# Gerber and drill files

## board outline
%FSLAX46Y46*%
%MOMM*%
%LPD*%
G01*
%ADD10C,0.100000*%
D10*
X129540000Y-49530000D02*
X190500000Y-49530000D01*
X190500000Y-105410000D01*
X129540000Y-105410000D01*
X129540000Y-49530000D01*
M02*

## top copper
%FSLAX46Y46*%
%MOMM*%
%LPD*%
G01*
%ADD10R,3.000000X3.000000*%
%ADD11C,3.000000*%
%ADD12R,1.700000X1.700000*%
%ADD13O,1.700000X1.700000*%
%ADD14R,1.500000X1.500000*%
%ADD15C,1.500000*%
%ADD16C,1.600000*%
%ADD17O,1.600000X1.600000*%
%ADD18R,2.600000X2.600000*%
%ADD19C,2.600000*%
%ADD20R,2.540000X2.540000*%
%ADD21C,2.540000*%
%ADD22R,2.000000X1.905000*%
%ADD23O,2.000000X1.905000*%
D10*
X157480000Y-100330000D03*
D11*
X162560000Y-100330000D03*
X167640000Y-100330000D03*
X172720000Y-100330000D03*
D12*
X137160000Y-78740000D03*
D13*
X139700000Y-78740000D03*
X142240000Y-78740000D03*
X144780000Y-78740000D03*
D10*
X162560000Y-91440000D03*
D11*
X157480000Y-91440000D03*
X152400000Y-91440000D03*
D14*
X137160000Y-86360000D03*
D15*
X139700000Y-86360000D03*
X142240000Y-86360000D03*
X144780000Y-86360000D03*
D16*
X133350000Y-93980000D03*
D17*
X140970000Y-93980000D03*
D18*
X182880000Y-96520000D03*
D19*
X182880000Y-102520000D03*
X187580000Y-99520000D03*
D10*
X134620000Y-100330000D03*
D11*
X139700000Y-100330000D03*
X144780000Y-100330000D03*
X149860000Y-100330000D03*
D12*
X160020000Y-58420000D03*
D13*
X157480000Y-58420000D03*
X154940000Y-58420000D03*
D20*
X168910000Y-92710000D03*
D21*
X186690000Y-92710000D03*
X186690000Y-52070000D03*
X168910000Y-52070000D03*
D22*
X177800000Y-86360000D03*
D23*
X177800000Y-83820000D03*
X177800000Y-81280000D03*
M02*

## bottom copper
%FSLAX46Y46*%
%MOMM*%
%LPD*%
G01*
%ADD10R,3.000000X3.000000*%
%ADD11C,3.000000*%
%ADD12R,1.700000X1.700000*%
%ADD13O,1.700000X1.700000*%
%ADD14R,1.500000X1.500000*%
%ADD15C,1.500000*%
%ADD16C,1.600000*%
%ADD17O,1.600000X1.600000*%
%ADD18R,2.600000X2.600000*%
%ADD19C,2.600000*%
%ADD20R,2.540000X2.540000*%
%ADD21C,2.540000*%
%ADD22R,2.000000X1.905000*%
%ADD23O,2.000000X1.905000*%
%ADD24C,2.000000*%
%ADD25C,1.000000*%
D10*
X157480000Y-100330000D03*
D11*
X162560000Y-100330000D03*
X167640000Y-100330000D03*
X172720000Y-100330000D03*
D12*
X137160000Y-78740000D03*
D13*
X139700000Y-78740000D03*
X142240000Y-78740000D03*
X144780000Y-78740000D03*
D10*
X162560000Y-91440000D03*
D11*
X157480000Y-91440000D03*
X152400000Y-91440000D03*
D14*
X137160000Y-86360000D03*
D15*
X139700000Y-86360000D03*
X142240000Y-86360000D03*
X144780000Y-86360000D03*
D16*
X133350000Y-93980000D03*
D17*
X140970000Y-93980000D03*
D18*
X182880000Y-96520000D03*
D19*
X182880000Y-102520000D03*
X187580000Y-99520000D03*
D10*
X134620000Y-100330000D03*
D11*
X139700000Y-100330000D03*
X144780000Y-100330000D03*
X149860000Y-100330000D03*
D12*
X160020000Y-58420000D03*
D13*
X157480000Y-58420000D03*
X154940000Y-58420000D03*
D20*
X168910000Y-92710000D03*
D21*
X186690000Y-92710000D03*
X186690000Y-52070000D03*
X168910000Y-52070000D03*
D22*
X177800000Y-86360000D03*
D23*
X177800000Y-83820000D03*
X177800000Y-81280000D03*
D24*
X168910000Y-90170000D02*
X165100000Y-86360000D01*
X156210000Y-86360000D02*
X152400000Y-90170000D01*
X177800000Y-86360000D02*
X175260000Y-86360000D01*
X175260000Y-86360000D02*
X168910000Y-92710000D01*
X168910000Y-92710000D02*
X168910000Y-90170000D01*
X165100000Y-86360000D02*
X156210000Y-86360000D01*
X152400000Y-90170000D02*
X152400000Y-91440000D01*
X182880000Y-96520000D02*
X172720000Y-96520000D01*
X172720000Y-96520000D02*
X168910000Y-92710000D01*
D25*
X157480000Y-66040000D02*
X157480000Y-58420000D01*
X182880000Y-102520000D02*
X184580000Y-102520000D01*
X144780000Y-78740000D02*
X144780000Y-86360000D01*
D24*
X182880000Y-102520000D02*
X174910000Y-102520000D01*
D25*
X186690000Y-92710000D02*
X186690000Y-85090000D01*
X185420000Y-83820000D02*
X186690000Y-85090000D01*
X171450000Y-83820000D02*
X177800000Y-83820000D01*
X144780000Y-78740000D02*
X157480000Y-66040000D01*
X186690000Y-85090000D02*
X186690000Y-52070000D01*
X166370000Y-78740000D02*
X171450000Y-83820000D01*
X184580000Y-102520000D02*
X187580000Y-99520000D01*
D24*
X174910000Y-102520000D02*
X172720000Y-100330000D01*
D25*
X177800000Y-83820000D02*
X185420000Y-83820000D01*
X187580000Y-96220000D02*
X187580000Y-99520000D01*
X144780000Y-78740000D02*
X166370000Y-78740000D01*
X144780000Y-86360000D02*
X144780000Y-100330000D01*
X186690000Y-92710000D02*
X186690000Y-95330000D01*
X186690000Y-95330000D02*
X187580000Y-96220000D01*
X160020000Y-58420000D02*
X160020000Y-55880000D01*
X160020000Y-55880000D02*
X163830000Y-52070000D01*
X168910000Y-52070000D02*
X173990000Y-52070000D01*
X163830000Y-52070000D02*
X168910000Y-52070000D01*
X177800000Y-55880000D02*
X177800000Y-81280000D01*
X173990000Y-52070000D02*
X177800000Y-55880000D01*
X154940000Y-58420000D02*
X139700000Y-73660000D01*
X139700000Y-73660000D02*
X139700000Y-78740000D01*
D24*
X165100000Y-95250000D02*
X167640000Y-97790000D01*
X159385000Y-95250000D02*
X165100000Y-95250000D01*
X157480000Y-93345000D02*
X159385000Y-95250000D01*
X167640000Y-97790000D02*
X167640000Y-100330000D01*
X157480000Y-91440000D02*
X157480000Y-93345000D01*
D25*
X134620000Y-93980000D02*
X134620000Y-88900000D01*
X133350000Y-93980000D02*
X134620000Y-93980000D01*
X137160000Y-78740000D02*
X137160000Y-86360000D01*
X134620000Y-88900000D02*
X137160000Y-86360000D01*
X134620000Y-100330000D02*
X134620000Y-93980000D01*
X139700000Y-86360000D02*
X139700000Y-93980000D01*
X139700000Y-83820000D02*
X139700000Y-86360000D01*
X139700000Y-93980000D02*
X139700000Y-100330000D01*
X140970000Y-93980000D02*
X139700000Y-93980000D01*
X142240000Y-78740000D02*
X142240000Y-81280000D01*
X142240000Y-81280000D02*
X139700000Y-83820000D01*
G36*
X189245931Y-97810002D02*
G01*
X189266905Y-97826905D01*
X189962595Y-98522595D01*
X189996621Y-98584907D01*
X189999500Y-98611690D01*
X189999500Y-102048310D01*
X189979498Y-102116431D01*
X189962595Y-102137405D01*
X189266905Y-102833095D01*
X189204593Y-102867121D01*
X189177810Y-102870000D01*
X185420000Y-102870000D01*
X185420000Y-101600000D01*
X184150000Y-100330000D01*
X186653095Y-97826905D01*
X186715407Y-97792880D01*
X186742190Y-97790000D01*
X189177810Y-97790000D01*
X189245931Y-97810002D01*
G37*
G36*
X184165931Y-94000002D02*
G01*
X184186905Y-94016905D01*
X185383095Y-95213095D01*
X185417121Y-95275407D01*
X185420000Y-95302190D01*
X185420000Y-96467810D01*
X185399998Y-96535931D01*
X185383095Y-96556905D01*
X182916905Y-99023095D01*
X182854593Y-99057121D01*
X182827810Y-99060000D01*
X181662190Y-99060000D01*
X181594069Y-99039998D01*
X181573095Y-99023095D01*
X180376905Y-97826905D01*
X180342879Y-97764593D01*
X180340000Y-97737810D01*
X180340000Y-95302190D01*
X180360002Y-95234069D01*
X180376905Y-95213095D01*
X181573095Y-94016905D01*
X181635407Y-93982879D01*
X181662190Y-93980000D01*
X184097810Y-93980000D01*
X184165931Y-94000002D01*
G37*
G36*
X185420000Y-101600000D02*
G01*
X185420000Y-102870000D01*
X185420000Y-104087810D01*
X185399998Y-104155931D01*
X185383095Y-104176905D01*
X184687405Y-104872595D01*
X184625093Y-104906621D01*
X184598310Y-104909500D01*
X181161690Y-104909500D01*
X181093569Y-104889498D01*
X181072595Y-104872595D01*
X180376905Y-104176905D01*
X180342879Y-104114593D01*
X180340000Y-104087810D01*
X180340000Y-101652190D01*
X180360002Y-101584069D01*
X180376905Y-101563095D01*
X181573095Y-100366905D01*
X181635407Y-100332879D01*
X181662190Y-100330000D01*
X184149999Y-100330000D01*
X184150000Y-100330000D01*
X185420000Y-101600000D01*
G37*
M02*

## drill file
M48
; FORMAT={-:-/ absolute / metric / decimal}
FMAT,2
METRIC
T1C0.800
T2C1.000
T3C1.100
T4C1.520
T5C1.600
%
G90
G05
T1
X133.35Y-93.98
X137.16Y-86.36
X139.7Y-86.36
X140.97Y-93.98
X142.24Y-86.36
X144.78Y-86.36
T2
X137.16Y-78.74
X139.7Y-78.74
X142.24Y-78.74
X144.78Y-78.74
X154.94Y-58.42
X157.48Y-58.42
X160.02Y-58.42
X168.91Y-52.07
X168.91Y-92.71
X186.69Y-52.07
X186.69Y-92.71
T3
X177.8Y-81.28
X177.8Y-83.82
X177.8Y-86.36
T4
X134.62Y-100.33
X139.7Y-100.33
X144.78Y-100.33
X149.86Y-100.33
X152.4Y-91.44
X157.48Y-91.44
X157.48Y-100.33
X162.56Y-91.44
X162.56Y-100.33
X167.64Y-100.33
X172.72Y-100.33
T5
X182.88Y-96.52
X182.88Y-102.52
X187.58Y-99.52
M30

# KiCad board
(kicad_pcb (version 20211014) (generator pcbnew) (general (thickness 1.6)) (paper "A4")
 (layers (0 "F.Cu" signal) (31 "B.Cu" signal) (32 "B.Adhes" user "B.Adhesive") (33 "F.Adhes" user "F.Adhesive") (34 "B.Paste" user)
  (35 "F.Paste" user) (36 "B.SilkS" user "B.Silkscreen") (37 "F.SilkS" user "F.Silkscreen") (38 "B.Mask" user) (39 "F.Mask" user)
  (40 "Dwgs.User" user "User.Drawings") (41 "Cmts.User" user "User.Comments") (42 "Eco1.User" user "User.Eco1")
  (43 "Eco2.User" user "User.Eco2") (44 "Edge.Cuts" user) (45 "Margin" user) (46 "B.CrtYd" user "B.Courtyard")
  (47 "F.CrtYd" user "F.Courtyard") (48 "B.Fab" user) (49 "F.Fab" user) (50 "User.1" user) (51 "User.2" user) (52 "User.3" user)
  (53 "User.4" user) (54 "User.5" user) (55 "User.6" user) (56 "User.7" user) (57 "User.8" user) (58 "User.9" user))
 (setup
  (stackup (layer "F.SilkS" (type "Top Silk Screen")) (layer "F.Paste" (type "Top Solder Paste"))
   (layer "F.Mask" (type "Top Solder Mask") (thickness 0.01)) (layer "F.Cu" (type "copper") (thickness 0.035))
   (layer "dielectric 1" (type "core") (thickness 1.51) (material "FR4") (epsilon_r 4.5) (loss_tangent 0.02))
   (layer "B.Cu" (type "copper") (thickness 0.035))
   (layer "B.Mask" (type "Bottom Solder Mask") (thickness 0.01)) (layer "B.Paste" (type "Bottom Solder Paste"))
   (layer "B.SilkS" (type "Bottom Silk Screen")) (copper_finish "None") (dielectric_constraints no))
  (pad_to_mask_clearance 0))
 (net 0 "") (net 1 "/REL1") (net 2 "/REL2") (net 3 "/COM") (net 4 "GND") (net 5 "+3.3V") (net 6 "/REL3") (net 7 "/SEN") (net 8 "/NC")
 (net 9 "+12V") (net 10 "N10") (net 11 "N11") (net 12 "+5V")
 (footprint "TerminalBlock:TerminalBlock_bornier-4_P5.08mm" (layer "F.Cu") (at 157.48 100.33)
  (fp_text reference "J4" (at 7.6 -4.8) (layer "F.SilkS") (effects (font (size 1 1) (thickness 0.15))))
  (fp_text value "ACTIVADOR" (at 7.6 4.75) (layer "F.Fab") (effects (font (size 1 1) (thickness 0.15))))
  (pad "1" thru_hole rect (at 0 0) (size 3 3) (drill 1.52) (layers *.Cu *.Mask) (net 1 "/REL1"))
  (pad "2" thru_hole circle (at 5.08 0) (size 3 3) (drill 1.52) (layers *.Cu *.Mask) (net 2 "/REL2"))
  (pad "3" thru_hole circle (at 10.16 0) (size 3 3) (drill 1.52) (layers *.Cu *.Mask) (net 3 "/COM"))
  (pad "4" thru_hole circle (at 15.24 0) (size 3 3) (drill 1.52) (layers *.Cu *.Mask) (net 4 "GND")))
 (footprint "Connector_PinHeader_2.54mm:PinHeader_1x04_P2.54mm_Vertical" (layer "F.Cu") (at 137.16 78.74 90)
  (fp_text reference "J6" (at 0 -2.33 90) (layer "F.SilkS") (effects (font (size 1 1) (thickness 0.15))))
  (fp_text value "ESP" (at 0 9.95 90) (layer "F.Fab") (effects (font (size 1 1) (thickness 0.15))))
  (pad "1" thru_hole rect (at 0 0 90) (size 1.7 1.7) (drill 1) (layers *.Cu *.Mask) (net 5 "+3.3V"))
  (pad "2" thru_hole oval (at 0 2.54 90) (size 1.7 1.7) (drill 1) (layers *.Cu *.Mask) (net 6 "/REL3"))
  (pad "3" thru_hole oval (at 0 5.08 90) (size 1.7 1.7) (drill 1) (layers *.Cu *.Mask) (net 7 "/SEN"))
  (pad "4" thru_hole oval (at 0 7.62 90) (size 1.7 1.7) (drill 1) (layers *.Cu *.Mask) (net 4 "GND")))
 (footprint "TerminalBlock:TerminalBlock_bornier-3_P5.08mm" (layer "F.Cu") (at 162.56 91.44 180)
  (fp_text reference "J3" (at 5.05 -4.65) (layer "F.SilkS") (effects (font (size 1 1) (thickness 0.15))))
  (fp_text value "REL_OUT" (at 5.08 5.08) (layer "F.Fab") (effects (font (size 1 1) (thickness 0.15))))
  (pad "1" thru_hole rect (at 0 0 180) (size 3 3) (drill 1.52) (layers *.Cu *.Mask) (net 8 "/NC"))
  (pad "2" thru_hole circle (at 5.08 0 180) (size 3 3) (drill 1.52) (layers *.Cu *.Mask) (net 3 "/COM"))
  (pad "3" thru_hole circle (at 10.16 0 180) (size 3 3) (drill 1.52) (layers *.Cu *.Mask) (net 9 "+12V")))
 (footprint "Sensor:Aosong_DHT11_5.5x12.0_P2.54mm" (layer "F.Cu") (at 137.16 86.36 90)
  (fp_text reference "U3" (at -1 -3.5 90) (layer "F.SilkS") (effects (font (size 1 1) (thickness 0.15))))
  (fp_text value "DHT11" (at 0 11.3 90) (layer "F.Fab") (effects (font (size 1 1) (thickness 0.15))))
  (pad "1" thru_hole rect (at 0 0 90) (size 1.5 1.5) (drill 0.8) (layers *.Cu *.Mask) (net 5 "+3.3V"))
  (pad "2" thru_hole circle (at 0 2.54 90) (size 1.5 1.5) (drill 0.8) (layers *.Cu *.Mask) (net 7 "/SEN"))
  (pad "3" thru_hole circle (at 0 5.08 90) (size 1.5 1.5) (drill 0.8) (layers *.Cu *.Mask) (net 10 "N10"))
  (pad "4" thru_hole circle (at 0 7.62 90) (size 1.5 1.5) (drill 0.8) (layers *.Cu *.Mask) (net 4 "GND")))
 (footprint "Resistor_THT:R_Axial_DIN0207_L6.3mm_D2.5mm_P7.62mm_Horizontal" (layer "F.Cu") (at 133.35 93.98)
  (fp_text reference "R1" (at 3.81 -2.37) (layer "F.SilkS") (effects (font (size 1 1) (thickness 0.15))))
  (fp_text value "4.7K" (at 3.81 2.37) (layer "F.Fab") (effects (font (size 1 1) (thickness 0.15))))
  (pad "1" thru_hole circle (at 0 0) (size 1.6 1.6) (drill 0.8) (layers *.Cu *.Mask) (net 5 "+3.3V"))
  (pad "2" thru_hole oval (at 7.62 0) (size 1.6 1.6) (drill 0.8) (layers *.Cu *.Mask) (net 7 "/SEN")))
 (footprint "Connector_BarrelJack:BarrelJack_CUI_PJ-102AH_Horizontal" (layer "F.Cu") (at 182.88 96.52)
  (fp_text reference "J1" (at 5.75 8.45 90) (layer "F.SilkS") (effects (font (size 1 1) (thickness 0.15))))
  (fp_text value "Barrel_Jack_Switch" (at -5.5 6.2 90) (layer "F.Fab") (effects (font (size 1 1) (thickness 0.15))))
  (pad "1" thru_hole rect (at 0 0) (size 2.6 2.6) (drill 1.6) (layers *.Cu *.Mask) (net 9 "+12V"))
  (pad "2" thru_hole circle (at 0 6) (size 2.6 2.6) (drill 1.6) (layers *.Cu *.Mask) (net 4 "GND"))
  (pad "3" thru_hole circle (at 4.7 3) (size 2.6 2.6) (drill 1.6) (layers *.Cu *.Mask) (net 4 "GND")))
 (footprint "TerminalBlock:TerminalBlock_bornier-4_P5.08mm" (layer "F.Cu") (at 134.62 100.33)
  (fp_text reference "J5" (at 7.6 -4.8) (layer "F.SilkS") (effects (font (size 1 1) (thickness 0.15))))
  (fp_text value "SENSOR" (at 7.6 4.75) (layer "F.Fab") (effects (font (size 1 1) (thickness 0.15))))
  (pad "1" thru_hole rect (at 0 0) (size 3 3) (drill 1.52) (layers *.Cu *.Mask) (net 5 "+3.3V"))
  (pad "2" thru_hole circle (at 5.08 0) (size 3 3) (drill 1.52) (layers *.Cu *.Mask) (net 7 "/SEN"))
  (pad "3" thru_hole circle (at 10.16 0) (size 3 3) (drill 1.52) (layers *.Cu *.Mask) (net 4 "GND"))
  (pad "4" thru_hole circle (at 15.24 0) (size 3 3) (drill 1.52) (layers *.Cu *.Mask) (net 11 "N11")))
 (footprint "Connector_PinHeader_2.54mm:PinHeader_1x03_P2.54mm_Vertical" (layer "F.Cu") (at 160.02 58.42 -90)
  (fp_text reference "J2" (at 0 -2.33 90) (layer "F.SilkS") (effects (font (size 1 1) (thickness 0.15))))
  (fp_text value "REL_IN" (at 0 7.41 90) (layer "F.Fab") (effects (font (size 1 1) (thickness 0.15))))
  (pad "1" thru_hole rect (at 0 0 270) (size 1.7 1.7) (drill 1) (layers *.Cu *.Mask) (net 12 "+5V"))
  (pad "2" thru_hole oval (at 0 2.54 270) (size 1.7 1.7) (drill 1) (layers *.Cu *.Mask) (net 4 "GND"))
  (pad "3" thru_hole oval (at 0 5.08 270) (size 1.7 1.7) (drill 1) (layers *.Cu *.Mask) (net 6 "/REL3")))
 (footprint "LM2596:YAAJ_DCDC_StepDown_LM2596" (layer "F.Cu") (at 168.91 92.71 90)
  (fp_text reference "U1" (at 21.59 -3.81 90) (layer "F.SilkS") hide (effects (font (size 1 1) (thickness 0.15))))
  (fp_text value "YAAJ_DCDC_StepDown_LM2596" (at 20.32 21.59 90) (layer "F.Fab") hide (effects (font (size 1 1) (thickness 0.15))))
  (pad "1" thru_hole rect locked (at 0 0 90) (size 2.54 2.54) (drill 1) (layers *.Cu *.Mask) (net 9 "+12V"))
  (pad "2" thru_hole circle locked (at 0 17.78 90) (size 2.54 2.54) (drill 1) (layers *.Cu *.Mask) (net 4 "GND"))
  (pad "3" thru_hole circle locked (at 40.64 17.78 90) (size 2.54 2.54) (drill 1) (layers *.Cu *.Mask) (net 4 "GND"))
  (pad "4" thru_hole circle locked (at 40.64 0 90) (size 2.54 2.54) (drill 1) (layers *.Cu *.Mask) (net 12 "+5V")))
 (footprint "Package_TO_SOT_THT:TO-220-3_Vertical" (layer "F.Cu") (at 177.8 86.36 90)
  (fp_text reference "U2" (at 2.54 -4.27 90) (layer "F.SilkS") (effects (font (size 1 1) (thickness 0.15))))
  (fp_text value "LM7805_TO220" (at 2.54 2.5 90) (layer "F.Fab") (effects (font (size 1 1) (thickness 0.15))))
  (pad "1" thru_hole rect (at 0 0 90) (size 1.905 2) (drill 1.1) (layers *.Cu *.Mask) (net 9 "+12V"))
  (pad "2" thru_hole oval (at 2.54 0 90) (size 1.905 2) (drill 1.1) (layers *.Cu *.Mask) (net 4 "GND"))
  (pad "3" thru_hole oval (at 5.08 0 90) (size 1.905 2) (drill 1.1) (layers *.Cu *.Mask) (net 12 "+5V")))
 (gr_rect (start 190.5 105.41) (end 129.54 49.53) (layer "Edge.Cuts") (width 0.1) (fill none))
 (segment (start 168.91 90.17) (end 165.1 86.36) (width 2) (layer "B.Cu") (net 9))
 (segment (start 156.21 86.36) (end 152.4 90.17) (width 2) (layer "B.Cu") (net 9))
 (segment (start 177.8 86.36) (end 175.26 86.36) (width 2) (layer "B.Cu") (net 9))
 (segment (start 175.26 86.36) (end 168.91 92.71) (width 2) (layer "B.Cu") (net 9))
 (segment (start 168.91 92.71) (end 168.91 90.17) (width 2) (layer "B.Cu") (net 9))
 (segment (start 165.1 86.36) (end 156.21 86.36) (width 2) (layer "B.Cu") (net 9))
 (segment (start 152.4 90.17) (end 152.4 91.44) (width 2) (layer "B.Cu") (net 9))
 (segment (start 182.88 96.52) (end 172.72 96.52) (width 2) (layer "B.Cu") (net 9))
 (segment (start 172.72 96.52) (end 168.91 92.71) (width 2) (layer "B.Cu") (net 9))
 (segment (start 157.48 66.04) (end 157.48 58.42) (width 1) (layer "B.Cu") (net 4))
 (segment (start 182.88 102.52) (end 184.58 102.52) (width 1) (layer "B.Cu") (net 4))
 (segment (start 144.78 78.74) (end 144.78 86.36) (width 1) (layer "B.Cu") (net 4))
 (segment (start 182.88 102.52) (end 174.91 102.52) (width 2) (layer "B.Cu") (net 4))
 (segment (start 186.69 92.71) (end 186.69 85.09) (width 1) (layer "B.Cu") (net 4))
 (segment (start 185.42 83.82) (end 186.69 85.09) (width 1) (layer "B.Cu") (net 4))
 (segment (start 171.45 83.82) (end 177.8 83.82) (width 1) (layer "B.Cu") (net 4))
 (segment (start 144.78 78.74) (end 157.48 66.04) (width 1) (layer "B.Cu") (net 4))
 (segment (start 186.69 85.09) (end 186.69 52.07) (width 1) (layer "B.Cu") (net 4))
 (segment (start 166.37 78.74) (end 171.45 83.82) (width 1) (layer "B.Cu") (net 4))
 (segment (start 184.58 102.52) (end 187.58 99.52) (width 1) (layer "B.Cu") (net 4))
 (segment (start 174.91 102.52) (end 172.72 100.33) (width 2) (layer "B.Cu") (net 4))
 (segment (start 177.8 83.82) (end 185.42 83.82) (width 1) (layer "B.Cu") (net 4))
 (segment (start 187.58 96.22) (end 187.58 99.52) (width 1) (layer "B.Cu") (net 4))
 (segment (start 144.78 78.74) (end 166.37 78.74) (width 1) (layer "B.Cu") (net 4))
 (segment (start 144.78 86.36) (end 144.78 100.33) (width 1) (layer "B.Cu") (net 4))
 (segment (start 186.69 92.71) (end 186.69 95.33) (width 1) (layer "B.Cu") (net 4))
 (segment (start 186.69 95.33) (end 187.58 96.22) (width 1) (layer "B.Cu") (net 4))
 (segment (start 160.02 58.42) (end 160.02 55.88) (width 1) (layer "B.Cu") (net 12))
 (segment (start 160.02 55.88) (end 163.83 52.07) (width 1) (layer "B.Cu") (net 12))
 (segment (start 168.91 52.07) (end 173.99 52.07) (width 1) (layer "B.Cu") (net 12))
 (segment (start 163.83 52.07) (end 168.91 52.07) (width 1) (layer "B.Cu") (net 12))
 (segment (start 177.8 55.88) (end 177.8 81.28) (width 1) (layer "B.Cu") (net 12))
 (segment (start 173.99 52.07) (end 177.8 55.88) (width 1) (layer "B.Cu") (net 12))
 (segment (start 154.94 58.42) (end 139.7 73.66) (width 1) (layer "B.Cu") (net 6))
 (segment (start 139.7 73.66) (end 139.7 78.74) (width 1) (layer "B.Cu") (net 6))
 (segment (start 165.1 95.25) (end 167.64 97.79) (width 2) (layer "B.Cu") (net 3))
 (segment (start 159.385 95.25) (end 165.1 95.25) (width 2) (layer "B.Cu") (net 3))
 (segment (start 157.48 93.345) (end 159.385 95.25) (width 2) (layer "B.Cu") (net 3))
 (segment (start 167.64 97.79) (end 167.64 100.33) (width 2) (layer "B.Cu") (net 3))
 (segment (start 157.48 91.44) (end 157.48 93.345) (width 2) (layer "B.Cu") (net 3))
 (segment (start 134.62 93.98) (end 134.62 88.9) (width 1) (layer "B.Cu") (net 5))
 (segment (start 133.35 93.98) (end 134.62 93.98) (width 1) (layer "B.Cu") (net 5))
 (segment (start 137.16 78.74) (end 137.16 86.36) (width 1) (layer "B.Cu") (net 5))
 (segment (start 134.62 88.9) (end 137.16 86.36) (width 1) (layer "B.Cu") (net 5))
 (segment (start 134.62 100.33) (end 134.62 93.98) (width 1) (layer "B.Cu") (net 5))
 (segment (start 139.7 86.36) (end 139.7 93.98) (width 1) (layer "B.Cu") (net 7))
 (segment (start 139.7 83.82) (end 139.7 86.36) (width 1) (layer "B.Cu") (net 7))
 (segment (start 139.7 93.98) (end 139.7 100.33) (width 1) (layer "B.Cu") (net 7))
 (segment (start 140.97 93.98) (end 139.7 93.98) (width 1) (layer "B.Cu") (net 7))
 (segment (start 142.24 78.74) (end 142.24 81.28) (width 1) (layer "B.Cu") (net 7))
 (segment (start 142.24 81.28) (end 139.7 83.82) (width 1) (layer "B.Cu") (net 7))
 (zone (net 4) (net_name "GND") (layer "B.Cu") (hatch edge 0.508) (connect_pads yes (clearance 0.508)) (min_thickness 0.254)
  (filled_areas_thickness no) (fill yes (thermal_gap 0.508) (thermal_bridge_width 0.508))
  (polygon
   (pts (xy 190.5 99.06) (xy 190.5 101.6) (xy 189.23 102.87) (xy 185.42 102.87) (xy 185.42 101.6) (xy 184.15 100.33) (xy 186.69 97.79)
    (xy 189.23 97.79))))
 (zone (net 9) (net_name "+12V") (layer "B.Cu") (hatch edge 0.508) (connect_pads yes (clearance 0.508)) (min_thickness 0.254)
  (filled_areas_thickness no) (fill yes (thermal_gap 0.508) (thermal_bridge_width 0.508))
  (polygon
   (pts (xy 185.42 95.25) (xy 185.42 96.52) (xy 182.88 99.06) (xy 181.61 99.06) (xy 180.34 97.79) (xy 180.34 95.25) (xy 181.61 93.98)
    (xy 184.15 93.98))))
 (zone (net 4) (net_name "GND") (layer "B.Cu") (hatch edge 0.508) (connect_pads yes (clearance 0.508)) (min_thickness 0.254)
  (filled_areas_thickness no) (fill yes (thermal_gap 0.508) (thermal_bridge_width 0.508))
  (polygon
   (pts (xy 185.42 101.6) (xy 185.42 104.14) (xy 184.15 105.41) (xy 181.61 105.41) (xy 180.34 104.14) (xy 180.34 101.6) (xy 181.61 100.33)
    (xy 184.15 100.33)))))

